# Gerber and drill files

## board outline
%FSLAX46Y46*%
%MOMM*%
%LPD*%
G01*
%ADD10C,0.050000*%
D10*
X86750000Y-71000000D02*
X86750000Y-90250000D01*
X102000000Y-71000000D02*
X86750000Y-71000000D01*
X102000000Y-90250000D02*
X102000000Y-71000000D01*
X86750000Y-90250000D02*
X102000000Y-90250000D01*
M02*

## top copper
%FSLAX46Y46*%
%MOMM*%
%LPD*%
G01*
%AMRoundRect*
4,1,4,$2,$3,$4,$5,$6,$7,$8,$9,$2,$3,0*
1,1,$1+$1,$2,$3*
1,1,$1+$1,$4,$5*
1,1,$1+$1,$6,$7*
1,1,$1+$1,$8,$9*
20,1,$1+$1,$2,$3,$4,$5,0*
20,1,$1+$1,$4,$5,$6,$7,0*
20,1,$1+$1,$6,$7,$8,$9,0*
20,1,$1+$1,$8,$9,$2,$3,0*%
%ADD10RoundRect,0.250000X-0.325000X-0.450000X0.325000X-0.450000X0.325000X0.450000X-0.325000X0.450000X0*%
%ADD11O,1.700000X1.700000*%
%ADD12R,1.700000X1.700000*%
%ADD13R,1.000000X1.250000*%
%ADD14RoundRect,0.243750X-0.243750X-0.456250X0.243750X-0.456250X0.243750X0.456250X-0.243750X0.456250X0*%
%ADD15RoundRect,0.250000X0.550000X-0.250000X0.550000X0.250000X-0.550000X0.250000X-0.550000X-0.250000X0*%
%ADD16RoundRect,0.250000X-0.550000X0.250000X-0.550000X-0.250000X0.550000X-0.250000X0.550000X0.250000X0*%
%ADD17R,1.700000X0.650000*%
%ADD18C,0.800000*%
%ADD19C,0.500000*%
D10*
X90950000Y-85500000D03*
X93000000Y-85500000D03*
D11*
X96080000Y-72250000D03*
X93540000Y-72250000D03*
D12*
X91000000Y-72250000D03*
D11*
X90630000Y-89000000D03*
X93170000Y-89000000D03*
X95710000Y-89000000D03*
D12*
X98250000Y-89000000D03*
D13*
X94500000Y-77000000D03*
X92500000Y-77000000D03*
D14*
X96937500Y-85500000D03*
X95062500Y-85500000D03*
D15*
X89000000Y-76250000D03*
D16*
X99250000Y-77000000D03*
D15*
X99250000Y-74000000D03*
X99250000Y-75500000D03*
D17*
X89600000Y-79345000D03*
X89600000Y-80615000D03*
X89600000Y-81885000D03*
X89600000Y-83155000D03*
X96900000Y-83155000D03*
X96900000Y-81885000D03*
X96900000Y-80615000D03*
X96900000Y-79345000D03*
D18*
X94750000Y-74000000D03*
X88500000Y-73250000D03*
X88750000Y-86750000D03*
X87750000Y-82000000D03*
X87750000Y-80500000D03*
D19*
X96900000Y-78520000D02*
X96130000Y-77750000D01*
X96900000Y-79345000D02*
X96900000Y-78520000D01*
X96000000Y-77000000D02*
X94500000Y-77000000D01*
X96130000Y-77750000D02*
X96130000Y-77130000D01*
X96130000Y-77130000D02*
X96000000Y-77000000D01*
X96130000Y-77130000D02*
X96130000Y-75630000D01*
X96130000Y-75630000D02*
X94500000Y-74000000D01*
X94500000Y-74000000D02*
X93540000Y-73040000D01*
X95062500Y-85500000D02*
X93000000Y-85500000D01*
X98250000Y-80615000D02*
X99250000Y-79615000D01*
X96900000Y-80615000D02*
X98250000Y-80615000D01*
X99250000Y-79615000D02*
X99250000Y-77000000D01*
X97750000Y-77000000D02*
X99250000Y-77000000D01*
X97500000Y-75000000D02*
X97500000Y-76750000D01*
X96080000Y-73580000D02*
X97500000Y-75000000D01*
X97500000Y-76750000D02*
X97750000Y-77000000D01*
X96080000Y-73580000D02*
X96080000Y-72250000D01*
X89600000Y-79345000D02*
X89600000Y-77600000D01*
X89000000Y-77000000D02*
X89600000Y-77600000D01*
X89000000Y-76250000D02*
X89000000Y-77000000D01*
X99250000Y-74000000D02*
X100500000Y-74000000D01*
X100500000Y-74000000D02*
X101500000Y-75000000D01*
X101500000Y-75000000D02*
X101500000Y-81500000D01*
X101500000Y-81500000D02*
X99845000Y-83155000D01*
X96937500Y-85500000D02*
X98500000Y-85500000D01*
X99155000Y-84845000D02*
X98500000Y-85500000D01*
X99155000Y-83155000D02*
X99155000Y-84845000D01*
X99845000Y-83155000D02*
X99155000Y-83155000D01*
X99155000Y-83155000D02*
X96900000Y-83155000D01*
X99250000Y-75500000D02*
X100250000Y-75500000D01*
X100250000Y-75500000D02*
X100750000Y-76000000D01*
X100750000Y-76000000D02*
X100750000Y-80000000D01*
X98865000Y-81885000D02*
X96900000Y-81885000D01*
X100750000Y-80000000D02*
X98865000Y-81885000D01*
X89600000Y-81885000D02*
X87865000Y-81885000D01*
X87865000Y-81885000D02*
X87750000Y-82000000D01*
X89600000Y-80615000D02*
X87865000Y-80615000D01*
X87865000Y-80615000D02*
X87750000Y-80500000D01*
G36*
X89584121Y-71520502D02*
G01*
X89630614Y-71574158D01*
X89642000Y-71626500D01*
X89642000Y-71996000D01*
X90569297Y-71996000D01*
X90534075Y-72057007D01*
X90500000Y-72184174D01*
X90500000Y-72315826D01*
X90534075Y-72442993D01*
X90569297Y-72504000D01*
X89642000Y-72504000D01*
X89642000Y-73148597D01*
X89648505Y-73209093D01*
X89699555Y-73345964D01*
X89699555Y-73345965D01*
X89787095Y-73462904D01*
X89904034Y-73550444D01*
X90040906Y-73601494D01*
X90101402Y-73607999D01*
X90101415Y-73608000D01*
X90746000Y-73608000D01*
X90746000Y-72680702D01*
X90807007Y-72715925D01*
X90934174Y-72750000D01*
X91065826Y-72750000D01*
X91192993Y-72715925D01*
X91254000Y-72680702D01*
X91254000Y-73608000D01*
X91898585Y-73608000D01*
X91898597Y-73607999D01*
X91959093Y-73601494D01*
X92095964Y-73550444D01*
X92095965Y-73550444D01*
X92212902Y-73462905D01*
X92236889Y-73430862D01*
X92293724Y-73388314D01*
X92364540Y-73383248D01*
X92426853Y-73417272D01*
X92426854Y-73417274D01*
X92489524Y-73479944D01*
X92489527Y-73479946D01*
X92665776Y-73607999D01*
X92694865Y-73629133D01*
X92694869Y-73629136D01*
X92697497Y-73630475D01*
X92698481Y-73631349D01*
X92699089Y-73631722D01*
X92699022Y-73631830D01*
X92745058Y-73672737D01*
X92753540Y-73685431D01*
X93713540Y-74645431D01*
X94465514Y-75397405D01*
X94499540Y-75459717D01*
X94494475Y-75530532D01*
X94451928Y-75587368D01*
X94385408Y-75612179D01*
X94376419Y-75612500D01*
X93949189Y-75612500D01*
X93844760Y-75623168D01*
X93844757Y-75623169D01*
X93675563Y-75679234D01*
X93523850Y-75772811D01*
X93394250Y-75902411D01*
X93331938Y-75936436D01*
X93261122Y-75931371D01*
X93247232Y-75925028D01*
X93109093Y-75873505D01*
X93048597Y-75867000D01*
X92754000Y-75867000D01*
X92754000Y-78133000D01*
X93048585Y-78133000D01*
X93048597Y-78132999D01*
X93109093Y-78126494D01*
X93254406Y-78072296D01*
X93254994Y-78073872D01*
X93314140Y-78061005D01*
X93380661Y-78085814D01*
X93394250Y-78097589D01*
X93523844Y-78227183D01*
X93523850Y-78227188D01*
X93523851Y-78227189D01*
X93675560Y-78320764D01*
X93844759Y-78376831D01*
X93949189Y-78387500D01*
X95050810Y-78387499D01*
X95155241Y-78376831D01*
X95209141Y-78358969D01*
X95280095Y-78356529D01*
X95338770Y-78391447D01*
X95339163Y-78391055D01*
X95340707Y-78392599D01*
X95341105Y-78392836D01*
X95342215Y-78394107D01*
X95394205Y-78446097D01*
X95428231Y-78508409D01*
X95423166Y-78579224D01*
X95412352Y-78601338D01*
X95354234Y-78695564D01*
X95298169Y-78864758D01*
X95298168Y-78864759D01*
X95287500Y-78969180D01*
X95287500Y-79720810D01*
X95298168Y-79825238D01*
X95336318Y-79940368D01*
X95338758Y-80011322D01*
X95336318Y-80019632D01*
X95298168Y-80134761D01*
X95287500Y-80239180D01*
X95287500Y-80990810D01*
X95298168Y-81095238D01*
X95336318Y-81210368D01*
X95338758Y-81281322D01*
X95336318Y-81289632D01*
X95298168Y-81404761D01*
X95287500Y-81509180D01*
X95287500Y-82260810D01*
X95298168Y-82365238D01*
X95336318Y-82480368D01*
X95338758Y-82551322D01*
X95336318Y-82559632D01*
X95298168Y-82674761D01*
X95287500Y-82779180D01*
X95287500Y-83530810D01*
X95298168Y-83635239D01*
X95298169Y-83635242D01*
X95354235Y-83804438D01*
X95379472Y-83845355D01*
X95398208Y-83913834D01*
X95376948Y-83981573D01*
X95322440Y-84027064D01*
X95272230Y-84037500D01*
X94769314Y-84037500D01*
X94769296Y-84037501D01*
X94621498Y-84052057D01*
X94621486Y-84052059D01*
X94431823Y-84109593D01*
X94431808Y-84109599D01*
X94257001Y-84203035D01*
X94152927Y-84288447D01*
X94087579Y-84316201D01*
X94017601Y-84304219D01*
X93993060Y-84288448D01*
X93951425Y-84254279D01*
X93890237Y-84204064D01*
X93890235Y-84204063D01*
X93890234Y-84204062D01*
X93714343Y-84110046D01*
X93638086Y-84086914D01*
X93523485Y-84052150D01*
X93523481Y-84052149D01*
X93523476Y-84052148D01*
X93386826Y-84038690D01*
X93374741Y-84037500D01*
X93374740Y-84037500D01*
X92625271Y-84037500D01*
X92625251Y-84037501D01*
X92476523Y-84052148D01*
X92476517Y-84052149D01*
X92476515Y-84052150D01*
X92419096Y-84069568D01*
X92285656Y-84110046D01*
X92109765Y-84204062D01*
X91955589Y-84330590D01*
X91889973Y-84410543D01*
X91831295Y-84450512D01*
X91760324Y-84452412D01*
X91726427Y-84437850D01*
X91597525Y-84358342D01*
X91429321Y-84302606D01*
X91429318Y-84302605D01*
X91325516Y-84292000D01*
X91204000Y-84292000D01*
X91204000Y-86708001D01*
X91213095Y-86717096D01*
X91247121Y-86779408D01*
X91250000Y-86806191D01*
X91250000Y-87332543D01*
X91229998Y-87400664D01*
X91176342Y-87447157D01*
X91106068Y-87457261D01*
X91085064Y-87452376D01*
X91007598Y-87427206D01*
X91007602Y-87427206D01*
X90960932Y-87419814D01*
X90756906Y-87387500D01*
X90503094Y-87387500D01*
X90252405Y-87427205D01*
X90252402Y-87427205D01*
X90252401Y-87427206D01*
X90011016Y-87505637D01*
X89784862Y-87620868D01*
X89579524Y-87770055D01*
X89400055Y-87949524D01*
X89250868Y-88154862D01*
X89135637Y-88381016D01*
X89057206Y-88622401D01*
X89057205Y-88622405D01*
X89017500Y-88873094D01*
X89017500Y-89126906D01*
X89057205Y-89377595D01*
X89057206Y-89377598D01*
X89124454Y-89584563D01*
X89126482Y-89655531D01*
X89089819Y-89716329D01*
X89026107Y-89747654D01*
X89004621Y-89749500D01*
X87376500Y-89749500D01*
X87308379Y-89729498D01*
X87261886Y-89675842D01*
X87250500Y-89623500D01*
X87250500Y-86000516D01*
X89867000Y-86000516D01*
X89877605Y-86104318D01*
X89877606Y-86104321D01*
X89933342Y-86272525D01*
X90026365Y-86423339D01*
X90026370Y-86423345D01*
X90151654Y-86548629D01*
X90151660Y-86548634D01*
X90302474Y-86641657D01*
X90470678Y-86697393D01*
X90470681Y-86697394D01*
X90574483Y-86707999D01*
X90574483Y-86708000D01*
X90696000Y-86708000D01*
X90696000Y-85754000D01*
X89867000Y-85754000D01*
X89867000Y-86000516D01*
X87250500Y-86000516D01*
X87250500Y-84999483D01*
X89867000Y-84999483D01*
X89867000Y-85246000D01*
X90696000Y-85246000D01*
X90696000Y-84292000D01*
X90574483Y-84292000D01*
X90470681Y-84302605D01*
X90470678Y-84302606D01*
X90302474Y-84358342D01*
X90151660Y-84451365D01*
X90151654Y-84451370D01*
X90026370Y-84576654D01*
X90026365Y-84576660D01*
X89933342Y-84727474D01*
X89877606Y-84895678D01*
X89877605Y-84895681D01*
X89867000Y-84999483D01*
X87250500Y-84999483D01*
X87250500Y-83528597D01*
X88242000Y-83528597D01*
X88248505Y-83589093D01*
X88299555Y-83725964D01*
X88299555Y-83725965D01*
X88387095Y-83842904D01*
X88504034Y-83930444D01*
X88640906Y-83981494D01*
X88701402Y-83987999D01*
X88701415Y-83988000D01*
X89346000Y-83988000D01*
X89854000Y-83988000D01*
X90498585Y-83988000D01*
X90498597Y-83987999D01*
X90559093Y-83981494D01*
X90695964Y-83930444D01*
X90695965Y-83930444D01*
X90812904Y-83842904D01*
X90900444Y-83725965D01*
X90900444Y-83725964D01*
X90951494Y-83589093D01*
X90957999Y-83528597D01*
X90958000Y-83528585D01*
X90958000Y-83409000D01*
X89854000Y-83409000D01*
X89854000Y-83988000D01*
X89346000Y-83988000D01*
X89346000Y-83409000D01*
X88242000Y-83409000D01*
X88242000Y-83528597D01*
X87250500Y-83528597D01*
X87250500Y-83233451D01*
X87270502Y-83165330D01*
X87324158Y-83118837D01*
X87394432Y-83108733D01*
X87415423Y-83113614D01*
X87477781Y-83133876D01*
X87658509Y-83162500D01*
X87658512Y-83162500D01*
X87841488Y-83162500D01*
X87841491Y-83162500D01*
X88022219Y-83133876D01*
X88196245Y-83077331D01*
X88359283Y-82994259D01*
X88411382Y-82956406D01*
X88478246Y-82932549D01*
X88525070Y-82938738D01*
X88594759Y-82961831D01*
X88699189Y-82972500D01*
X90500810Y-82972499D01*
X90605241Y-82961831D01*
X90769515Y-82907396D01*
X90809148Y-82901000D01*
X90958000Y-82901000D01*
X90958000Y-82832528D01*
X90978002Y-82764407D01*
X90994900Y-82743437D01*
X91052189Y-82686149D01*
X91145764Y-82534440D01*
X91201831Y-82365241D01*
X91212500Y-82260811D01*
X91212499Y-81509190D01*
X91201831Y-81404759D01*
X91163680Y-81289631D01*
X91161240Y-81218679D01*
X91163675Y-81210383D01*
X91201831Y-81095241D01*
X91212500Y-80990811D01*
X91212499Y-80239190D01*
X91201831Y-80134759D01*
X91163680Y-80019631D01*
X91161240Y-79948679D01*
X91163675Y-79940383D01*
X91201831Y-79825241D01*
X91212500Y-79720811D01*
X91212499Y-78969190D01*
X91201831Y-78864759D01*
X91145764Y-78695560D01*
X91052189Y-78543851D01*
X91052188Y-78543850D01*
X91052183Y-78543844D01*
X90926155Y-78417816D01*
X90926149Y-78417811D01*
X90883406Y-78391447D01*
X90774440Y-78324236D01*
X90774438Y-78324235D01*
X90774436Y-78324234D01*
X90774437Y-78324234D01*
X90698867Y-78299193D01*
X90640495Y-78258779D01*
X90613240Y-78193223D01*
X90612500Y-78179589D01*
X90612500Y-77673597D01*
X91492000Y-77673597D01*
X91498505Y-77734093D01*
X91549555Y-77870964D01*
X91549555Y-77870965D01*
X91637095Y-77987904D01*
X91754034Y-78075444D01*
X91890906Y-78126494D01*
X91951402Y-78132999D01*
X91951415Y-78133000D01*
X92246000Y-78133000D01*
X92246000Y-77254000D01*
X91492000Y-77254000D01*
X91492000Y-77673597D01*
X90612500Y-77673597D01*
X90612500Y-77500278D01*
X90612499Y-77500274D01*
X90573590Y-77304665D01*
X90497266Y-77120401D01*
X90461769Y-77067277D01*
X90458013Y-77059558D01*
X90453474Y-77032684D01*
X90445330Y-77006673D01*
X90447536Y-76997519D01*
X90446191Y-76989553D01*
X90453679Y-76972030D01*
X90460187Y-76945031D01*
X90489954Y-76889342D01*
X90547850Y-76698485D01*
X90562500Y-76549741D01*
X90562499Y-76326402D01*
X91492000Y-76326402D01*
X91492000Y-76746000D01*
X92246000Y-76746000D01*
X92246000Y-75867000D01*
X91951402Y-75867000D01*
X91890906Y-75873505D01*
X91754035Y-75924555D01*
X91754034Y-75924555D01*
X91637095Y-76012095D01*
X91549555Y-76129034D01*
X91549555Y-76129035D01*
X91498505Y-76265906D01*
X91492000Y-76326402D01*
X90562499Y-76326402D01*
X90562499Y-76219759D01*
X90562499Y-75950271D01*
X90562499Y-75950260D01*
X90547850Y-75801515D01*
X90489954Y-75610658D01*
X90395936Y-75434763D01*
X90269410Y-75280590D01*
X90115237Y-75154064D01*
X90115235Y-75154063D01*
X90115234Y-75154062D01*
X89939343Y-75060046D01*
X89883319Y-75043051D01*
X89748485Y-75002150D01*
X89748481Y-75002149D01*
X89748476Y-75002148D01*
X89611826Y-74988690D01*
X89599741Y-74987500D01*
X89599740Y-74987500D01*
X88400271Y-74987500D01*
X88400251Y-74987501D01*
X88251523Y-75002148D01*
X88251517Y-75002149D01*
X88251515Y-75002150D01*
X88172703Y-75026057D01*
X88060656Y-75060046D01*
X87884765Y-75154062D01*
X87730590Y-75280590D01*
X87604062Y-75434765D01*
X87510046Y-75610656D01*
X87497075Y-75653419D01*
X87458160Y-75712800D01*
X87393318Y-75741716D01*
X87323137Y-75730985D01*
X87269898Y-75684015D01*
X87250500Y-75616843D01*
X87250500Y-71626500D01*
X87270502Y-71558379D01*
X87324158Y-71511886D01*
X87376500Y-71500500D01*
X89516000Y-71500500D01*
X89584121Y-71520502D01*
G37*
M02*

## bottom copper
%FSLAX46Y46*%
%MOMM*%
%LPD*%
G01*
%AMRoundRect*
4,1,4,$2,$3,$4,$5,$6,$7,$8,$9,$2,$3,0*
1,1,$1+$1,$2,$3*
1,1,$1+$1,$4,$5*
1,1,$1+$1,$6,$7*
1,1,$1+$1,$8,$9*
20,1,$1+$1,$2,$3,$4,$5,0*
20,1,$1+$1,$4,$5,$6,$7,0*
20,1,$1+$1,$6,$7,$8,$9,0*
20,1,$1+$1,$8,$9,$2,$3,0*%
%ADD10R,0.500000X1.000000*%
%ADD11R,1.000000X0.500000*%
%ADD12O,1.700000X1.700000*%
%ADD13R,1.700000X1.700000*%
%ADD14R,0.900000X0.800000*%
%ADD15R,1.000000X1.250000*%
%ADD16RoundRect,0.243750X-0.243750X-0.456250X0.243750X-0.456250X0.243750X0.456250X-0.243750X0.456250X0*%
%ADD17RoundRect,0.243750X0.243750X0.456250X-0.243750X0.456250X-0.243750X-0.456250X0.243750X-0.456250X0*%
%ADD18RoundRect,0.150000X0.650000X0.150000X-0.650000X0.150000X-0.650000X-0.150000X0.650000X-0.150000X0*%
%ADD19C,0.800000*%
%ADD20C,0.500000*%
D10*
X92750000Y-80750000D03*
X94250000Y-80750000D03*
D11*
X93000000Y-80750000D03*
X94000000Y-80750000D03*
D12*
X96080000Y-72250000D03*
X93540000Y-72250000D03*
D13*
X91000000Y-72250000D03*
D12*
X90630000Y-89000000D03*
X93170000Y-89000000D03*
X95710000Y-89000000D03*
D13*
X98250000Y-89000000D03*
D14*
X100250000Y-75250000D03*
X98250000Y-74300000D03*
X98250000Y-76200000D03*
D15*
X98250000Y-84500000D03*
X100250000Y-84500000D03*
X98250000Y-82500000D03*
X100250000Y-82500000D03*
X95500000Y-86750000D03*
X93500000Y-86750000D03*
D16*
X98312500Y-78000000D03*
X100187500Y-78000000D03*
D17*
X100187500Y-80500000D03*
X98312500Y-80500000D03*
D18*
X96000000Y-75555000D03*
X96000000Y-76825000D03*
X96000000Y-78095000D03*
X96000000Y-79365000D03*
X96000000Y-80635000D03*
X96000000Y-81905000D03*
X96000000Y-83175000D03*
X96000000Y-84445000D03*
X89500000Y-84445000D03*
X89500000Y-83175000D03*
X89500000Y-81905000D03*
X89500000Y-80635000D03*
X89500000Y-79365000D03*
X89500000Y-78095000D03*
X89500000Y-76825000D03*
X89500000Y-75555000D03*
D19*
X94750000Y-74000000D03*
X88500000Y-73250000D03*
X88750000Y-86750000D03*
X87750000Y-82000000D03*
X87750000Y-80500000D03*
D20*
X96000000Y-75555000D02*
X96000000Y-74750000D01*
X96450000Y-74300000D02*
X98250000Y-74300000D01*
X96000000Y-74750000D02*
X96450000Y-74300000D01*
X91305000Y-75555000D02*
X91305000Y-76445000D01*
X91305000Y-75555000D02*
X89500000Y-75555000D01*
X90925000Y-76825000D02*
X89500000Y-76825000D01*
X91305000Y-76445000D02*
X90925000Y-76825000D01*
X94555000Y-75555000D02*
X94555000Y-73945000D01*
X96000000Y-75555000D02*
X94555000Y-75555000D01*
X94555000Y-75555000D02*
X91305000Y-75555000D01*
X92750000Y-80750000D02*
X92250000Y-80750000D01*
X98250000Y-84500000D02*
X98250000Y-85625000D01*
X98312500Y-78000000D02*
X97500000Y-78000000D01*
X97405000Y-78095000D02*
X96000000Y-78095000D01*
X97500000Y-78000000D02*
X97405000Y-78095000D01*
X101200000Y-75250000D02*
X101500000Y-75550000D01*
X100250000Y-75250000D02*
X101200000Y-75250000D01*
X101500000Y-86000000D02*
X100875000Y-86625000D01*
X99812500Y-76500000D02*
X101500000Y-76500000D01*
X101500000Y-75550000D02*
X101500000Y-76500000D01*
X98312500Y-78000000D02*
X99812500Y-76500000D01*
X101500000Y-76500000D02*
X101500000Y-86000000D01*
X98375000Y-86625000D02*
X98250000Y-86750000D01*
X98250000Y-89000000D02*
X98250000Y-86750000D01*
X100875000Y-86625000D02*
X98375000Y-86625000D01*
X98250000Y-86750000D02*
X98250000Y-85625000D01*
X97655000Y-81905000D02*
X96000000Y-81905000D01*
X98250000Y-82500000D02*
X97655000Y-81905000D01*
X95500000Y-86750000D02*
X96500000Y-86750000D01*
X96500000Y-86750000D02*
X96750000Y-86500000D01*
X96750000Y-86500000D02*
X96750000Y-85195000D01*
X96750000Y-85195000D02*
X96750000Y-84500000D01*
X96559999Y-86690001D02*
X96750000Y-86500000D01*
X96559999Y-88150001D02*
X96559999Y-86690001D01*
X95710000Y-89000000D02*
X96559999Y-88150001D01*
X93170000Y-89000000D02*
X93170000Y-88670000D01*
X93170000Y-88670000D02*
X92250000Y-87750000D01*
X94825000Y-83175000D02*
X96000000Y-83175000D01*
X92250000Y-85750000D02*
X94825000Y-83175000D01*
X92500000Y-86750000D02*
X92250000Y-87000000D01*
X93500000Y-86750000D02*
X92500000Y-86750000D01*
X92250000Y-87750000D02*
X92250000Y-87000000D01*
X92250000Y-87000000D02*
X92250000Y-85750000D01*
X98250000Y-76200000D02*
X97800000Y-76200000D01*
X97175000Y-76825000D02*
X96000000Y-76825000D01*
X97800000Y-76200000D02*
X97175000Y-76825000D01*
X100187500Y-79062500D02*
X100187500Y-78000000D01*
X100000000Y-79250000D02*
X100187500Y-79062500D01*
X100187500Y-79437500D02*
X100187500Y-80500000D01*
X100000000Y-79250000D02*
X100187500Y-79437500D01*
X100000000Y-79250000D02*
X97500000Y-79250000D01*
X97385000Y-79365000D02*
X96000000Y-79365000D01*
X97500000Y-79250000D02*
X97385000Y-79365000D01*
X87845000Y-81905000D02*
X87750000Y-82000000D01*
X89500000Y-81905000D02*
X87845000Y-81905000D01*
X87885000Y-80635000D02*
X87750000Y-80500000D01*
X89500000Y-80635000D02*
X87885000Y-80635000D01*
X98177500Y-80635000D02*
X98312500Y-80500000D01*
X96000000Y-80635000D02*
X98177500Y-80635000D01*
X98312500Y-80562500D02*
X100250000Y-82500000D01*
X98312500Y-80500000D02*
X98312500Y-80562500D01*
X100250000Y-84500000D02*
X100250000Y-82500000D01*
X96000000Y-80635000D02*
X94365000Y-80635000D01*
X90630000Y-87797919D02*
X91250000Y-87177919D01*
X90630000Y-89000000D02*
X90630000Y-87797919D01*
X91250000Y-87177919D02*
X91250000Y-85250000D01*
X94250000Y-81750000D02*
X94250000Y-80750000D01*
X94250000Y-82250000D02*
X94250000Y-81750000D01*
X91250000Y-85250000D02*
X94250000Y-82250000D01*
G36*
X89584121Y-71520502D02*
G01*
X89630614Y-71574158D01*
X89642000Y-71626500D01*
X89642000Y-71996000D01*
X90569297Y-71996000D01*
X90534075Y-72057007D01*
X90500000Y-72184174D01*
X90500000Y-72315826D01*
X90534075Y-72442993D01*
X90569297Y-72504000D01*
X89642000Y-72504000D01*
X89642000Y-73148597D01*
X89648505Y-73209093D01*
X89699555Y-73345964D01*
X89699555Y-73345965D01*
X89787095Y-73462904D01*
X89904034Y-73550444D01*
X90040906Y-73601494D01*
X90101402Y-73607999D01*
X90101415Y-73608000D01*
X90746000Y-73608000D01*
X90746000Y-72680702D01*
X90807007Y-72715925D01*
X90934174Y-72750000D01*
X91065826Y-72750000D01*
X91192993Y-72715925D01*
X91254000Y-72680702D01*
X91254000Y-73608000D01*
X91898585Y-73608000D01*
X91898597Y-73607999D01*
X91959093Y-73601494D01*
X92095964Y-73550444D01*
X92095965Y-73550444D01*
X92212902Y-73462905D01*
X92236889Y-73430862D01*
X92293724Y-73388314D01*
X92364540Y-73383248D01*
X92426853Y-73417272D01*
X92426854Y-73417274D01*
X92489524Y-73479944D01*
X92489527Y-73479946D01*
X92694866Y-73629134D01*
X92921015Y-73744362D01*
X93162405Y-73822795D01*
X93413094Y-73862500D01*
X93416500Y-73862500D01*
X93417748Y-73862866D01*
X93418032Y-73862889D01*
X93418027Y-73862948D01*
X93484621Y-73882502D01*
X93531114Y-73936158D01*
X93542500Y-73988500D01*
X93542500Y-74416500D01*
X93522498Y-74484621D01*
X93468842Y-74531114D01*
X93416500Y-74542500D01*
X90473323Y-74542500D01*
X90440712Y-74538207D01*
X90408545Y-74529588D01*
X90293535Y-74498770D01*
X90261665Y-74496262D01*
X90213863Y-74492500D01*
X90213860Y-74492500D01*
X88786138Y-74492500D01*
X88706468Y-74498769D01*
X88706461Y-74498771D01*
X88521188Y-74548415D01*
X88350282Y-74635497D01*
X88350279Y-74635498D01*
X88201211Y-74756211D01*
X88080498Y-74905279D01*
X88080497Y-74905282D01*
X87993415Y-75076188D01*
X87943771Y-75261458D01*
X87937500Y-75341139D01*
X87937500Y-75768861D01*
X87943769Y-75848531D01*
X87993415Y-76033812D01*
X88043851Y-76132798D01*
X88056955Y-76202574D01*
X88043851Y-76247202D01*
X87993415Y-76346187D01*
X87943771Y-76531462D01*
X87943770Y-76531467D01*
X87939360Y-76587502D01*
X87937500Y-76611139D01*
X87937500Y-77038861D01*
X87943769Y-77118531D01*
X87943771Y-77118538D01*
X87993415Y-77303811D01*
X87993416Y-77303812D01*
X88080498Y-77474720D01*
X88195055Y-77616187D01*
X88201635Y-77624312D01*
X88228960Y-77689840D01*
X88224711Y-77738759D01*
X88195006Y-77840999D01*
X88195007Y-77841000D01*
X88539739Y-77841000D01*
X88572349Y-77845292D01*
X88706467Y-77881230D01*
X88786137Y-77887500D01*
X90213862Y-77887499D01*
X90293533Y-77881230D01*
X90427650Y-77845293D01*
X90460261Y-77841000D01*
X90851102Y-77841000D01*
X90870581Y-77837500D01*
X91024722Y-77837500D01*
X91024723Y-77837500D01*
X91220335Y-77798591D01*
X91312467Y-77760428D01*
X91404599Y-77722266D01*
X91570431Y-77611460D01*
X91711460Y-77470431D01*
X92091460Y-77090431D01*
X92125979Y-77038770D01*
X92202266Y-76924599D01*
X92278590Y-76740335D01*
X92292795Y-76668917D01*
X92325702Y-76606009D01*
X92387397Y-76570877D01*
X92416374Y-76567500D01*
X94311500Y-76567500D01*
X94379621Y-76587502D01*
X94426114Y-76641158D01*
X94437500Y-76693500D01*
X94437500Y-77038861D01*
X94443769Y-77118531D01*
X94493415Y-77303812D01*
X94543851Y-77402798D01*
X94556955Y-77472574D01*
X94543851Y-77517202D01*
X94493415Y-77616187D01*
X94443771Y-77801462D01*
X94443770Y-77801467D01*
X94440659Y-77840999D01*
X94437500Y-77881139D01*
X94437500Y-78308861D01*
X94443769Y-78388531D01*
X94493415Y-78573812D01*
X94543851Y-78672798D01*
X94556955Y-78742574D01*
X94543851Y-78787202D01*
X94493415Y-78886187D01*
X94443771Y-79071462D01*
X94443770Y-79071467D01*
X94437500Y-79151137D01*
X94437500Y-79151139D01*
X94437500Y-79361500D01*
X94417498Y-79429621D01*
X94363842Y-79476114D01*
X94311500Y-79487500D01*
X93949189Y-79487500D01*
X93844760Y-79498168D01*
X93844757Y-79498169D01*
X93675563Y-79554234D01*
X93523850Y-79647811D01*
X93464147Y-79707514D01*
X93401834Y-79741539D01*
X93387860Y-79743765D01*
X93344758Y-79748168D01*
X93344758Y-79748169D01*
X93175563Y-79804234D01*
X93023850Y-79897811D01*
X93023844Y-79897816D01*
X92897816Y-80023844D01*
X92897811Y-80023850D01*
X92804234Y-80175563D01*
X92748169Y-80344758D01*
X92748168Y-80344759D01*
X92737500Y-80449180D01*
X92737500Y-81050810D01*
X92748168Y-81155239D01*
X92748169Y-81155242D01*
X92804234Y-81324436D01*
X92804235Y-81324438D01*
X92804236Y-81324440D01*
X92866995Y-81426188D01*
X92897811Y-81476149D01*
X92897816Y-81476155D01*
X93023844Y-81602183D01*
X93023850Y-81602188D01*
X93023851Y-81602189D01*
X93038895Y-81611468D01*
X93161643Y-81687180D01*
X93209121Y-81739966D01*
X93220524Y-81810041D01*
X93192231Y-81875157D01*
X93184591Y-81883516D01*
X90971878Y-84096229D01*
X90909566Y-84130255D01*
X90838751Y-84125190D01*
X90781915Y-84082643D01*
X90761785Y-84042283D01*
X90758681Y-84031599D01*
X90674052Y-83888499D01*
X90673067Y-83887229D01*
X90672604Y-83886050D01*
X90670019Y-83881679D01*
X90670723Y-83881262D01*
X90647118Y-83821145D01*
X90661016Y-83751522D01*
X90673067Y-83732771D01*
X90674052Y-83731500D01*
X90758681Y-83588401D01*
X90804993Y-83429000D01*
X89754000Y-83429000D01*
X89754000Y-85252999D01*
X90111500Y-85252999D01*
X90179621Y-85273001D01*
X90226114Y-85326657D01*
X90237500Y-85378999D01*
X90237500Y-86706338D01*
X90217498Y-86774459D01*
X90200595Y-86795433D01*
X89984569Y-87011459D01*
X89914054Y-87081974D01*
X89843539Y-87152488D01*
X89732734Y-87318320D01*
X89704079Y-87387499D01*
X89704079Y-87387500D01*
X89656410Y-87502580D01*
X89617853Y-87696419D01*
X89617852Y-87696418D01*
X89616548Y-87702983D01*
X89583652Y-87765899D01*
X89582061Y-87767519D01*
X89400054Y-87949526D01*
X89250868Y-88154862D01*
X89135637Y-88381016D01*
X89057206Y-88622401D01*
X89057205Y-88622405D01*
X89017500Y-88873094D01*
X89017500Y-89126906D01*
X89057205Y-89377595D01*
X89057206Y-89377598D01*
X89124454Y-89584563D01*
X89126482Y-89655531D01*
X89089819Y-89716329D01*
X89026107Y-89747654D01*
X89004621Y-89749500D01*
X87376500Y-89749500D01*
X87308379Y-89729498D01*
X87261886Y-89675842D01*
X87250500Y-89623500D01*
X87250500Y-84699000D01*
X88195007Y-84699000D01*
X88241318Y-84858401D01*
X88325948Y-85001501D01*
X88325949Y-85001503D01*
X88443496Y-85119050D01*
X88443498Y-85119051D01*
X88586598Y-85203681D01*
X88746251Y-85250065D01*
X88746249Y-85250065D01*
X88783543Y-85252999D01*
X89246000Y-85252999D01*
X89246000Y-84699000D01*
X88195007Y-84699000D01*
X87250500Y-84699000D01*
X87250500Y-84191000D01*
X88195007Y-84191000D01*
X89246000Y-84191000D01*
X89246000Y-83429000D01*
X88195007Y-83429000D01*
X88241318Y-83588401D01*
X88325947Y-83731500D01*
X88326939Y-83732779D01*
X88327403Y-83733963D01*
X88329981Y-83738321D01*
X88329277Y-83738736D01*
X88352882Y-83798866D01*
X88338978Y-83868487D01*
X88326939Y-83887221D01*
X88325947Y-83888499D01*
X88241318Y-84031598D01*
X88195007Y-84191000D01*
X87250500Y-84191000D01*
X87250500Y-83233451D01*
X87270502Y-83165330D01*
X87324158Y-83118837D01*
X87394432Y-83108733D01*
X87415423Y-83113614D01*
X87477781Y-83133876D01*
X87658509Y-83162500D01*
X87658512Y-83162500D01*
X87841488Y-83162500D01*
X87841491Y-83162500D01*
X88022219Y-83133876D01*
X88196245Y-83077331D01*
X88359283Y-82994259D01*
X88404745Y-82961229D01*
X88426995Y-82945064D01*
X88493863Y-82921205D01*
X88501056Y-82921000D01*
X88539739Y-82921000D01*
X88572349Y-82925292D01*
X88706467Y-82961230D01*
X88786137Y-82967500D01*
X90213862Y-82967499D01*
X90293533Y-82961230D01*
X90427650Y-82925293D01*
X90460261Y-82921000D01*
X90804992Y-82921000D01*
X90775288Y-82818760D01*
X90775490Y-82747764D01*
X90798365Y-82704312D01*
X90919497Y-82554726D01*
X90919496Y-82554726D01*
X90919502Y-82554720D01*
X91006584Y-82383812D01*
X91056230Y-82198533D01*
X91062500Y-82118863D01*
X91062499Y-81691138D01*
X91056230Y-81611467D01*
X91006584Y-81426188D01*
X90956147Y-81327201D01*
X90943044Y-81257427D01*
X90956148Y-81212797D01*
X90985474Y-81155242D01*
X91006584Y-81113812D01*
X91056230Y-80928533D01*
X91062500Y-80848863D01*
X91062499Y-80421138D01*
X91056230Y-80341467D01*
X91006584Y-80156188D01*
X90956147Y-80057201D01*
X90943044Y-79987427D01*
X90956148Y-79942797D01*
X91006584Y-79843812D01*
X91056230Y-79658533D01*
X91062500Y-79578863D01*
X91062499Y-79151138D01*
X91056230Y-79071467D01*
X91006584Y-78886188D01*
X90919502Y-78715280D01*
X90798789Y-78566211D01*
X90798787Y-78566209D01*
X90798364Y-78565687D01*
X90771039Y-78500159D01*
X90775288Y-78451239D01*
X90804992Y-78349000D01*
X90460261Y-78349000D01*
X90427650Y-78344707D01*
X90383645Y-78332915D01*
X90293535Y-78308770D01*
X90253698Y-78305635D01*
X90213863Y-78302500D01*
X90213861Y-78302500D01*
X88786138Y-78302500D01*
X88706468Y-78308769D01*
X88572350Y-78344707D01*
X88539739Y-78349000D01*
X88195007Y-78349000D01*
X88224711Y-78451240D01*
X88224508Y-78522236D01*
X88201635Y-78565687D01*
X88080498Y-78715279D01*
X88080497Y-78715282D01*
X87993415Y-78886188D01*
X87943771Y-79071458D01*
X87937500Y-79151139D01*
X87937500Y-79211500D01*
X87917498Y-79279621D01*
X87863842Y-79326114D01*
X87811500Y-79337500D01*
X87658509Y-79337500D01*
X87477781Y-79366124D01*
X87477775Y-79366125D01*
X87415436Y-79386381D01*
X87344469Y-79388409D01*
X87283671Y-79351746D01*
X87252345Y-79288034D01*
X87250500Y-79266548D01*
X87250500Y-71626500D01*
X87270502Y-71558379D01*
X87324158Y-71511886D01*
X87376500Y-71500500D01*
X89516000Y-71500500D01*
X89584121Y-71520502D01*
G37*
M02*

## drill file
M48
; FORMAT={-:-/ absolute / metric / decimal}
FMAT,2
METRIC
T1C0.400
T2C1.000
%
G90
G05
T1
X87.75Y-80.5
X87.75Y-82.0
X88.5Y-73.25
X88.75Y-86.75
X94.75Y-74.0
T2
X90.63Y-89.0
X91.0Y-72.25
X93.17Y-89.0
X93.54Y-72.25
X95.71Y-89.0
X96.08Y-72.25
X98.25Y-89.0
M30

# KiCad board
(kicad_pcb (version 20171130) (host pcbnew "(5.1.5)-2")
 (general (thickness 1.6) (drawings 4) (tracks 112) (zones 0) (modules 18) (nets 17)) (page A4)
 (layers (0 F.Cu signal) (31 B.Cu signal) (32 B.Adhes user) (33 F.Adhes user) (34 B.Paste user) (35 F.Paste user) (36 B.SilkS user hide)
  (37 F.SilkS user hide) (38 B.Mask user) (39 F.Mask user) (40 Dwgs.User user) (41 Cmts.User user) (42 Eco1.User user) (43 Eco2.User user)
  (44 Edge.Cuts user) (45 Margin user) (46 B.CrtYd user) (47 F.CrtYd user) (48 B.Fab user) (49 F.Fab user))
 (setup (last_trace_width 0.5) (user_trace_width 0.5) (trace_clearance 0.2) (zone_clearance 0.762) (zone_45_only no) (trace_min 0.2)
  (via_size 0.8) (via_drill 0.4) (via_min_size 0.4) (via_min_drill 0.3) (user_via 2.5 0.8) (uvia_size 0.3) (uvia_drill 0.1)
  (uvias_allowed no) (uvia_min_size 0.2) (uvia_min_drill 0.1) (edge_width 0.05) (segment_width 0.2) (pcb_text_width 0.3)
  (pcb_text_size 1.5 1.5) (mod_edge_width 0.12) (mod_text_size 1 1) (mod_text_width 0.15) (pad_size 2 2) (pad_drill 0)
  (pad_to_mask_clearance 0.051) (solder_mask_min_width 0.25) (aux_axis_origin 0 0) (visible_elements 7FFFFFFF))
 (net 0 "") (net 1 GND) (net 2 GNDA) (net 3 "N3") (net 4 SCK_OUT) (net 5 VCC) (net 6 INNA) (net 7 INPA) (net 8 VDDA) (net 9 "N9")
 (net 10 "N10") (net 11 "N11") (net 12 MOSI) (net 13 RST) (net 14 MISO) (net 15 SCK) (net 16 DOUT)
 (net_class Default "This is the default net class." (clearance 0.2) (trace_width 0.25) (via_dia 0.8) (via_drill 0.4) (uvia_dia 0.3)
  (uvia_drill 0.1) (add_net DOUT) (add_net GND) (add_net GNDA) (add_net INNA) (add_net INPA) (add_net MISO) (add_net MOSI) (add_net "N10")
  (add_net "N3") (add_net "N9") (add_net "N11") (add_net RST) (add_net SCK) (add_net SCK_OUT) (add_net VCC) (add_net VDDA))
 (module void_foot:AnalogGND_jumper (layer B.Cu) (at 93.5 80.75 180) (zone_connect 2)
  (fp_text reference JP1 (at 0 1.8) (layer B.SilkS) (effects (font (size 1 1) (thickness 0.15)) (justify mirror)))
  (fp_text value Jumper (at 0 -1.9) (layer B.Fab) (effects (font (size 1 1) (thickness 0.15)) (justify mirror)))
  (pad 2 smd rect (at 0.75 0 180) (size 0.5 1) (layers B.Cu B.Mask) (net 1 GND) (zone_connect 2))
  (pad 1 smd rect (at -0.75 0 180) (size 0.5 1) (layers B.Cu B.Mask) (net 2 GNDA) (zone_connect 2))
  (pad 2 smd rect (at 0.5 0 180) (size 1 0.5) (layers B.Cu B.Mask) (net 1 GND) (zone_connect 2))
  (pad 1 smd rect (at -0.5 0 180) (size 1 0.5) (layers B.Cu B.Mask) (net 2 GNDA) (zone_connect 2)))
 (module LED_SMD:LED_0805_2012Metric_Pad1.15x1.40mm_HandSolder (layer F.Cu) (at 91.975 85.5)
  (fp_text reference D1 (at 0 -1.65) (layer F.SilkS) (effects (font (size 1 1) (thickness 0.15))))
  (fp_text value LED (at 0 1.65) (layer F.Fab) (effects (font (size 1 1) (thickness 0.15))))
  (pad 1 smd roundrect (at -1.025 0) (size 1.15 1.4) (layers F.Cu F.Paste F.Mask) (roundrect_rratio 0.217391) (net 1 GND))
  (pad 2 smd roundrect (at 1.025 0) (size 1.15 1.4) (layers F.Cu F.Paste F.Mask) (roundrect_rratio 0.217391) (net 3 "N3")))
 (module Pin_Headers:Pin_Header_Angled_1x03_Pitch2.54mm (layer F.Cu) (at 91 72.25 90)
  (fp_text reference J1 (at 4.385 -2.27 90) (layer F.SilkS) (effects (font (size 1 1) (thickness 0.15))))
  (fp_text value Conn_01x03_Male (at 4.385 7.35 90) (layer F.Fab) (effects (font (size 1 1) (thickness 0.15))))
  (pad 3 thru_hole oval (at 0 5.08 90) (size 1.7 1.7) (drill 1) (layers *.Cu *.Mask) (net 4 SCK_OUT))
  (pad 2 thru_hole oval (at 0 2.54 90) (size 1.7 1.7) (drill 1) (layers *.Cu *.Mask) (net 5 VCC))
  (pad 1 thru_hole rect (at 0 0 90) (size 1.7 1.7) (drill 1) (layers *.Cu *.Mask) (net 1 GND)))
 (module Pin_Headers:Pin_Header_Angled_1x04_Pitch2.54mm (layer F.Cu) (at 98.25 89 270)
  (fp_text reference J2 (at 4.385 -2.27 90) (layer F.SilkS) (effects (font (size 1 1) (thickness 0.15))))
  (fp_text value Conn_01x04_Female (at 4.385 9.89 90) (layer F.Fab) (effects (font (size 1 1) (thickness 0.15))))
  (pad 4 thru_hole oval (at 0 7.62 270) (size 1.7 1.7) (drill 1) (layers *.Cu *.Mask) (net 2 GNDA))
  (pad 3 thru_hole oval (at 0 5.08 270) (size 1.7 1.7) (drill 1) (layers *.Cu *.Mask) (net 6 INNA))
  (pad 2 thru_hole oval (at 0 2.54 270) (size 1.7 1.7) (drill 1) (layers *.Cu *.Mask) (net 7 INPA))
  (pad 1 thru_hole rect (at 0 0 270) (size 1.7 1.7) (drill 1) (layers *.Cu *.Mask) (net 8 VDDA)))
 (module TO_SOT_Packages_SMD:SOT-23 (layer B.Cu) (at 99.25 75.25)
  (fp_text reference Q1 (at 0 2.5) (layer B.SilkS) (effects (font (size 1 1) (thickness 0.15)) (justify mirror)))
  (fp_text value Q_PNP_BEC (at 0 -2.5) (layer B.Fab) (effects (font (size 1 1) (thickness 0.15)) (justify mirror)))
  (pad 3 smd rect (at 1 0) (size 0.9 0.8) (layers B.Cu B.Paste B.Mask) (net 8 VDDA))
  (pad 2 smd rect (at -1 -0.95) (size 0.9 0.8) (layers B.Cu B.Paste B.Mask) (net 5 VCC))
  (pad 1 smd rect (at -1 0.95) (size 0.9 0.8) (layers B.Cu B.Paste B.Mask) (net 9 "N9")))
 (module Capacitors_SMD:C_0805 (layer F.Cu) (at 93.5 77 180)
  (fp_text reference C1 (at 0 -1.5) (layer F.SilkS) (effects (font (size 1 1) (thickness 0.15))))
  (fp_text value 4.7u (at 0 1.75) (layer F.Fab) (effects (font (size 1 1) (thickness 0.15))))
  (pad 1 smd rect (at -1 0 180) (size 1 1.25) (layers F.Cu F.Paste F.Mask) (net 5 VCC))
  (pad 2 smd rect (at 1 0 180) (size 1 1.25) (layers F.Cu F.Paste F.Mask) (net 1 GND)))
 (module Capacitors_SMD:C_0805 (layer B.Cu) (at 99.25 84.5)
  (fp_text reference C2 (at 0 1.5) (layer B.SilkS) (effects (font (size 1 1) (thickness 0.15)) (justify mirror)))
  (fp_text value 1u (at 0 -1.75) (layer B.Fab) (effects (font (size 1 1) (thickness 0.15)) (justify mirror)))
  (pad 1 smd rect (at -1 0) (size 1 1.25) (layers B.Cu B.Paste B.Mask) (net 8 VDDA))
  (pad 2 smd rect (at 1 0) (size 1 1.25) (layers B.Cu B.Paste B.Mask) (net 2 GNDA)))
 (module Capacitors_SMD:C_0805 (layer B.Cu) (at 99.25 82.5 180)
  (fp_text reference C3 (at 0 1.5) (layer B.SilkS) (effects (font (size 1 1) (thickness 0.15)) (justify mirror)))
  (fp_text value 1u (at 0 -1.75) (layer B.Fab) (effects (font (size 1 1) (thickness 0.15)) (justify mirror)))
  (pad 2 smd rect (at 1 0 180) (size 1 1.25) (layers B.Cu B.Paste B.Mask) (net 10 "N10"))
  (pad 1 smd rect (at -1 0 180) (size 1 1.25) (layers B.Cu B.Paste B.Mask) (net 2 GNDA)))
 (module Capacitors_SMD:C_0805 (layer B.Cu) (at 94.5 86.75)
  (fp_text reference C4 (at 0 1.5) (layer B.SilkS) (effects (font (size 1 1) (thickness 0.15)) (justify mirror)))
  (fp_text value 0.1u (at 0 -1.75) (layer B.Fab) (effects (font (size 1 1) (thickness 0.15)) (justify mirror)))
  (pad 2 smd rect (at 1 0) (size 1 1.25) (layers B.Cu B.Paste B.Mask) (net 7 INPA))
  (pad 1 smd rect (at -1 0) (size 1 1.25) (layers B.Cu B.Paste B.Mask) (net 6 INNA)))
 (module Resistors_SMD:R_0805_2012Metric (layer B.Cu) (at 99.25 78)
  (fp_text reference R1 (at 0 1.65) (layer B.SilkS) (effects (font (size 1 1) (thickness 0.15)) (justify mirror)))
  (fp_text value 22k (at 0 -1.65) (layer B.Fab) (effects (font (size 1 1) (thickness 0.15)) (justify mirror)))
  (pad 1 smd roundrect (at -0.9375 0) (size 0.975 1.4) (layers B.Cu B.Paste B.Mask) (roundrect_rratio 0.25) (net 8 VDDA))
  (pad 2 smd roundrect (at 0.9375 0) (size 0.975 1.4) (layers B.Cu B.Paste B.Mask) (roundrect_rratio 0.25) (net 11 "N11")))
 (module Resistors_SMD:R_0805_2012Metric (layer B.Cu) (at 99.25 80.5 180)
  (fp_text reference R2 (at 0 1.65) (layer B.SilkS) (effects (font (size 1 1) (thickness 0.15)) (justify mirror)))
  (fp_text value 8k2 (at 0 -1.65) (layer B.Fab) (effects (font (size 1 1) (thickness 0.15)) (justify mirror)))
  (pad 1 smd roundrect (at -0.9375 0 180) (size 0.975 1.4) (layers B.Cu B.Paste B.Mask) (roundrect_rratio 0.25) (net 11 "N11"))
  (pad 2 smd roundrect (at 0.9375 0 180) (size 0.975 1.4) (layers B.Cu B.Paste B.Mask) (roundrect_rratio 0.25) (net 2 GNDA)))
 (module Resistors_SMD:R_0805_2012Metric (layer F.Cu) (at 96 85.5)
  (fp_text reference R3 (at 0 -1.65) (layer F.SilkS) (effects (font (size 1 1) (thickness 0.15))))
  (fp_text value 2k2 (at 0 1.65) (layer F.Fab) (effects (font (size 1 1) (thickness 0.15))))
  (pad 2 smd roundrect (at 0.9375 0) (size 0.975 1.4) (layers F.Cu F.Paste F.Mask) (roundrect_rratio 0.25) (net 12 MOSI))
  (pad 1 smd roundrect (at -0.9375 0) (size 0.975 1.4) (layers F.Cu F.Paste F.Mask) (roundrect_rratio 0.25) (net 3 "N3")))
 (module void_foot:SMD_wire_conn (layer F.Cu) (at 89 76.25 90)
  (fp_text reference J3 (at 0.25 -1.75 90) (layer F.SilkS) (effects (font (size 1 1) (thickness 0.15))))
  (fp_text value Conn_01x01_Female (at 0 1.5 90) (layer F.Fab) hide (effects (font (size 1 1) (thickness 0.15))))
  (pad 1 smd roundrect (at 0 0 90) (size 1 1.6) (layers F.Cu F.Paste F.Mask) (roundrect_rratio 0.25) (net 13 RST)))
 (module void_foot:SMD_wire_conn (layer F.Cu) (at 99.25 77 270)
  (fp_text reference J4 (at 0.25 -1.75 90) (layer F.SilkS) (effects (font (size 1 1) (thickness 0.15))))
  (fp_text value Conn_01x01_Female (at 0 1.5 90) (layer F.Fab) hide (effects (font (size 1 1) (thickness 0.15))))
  (pad 1 smd roundrect (at 0 0 270) (size 1 1.6) (layers F.Cu F.Paste F.Mask) (roundrect_rratio 0.25) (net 4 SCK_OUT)))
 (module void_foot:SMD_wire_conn (layer F.Cu) (at 99.25 74 90)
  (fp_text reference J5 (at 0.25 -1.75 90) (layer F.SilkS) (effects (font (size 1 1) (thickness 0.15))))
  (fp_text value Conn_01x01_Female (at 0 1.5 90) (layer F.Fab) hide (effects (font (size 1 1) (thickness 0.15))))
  (pad 1 smd roundrect (at 0 0 90) (size 1 1.6) (layers F.Cu F.Paste F.Mask) (roundrect_rratio 0.25) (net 12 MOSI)))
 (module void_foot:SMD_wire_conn (layer F.Cu) (at 99.25 75.5 90)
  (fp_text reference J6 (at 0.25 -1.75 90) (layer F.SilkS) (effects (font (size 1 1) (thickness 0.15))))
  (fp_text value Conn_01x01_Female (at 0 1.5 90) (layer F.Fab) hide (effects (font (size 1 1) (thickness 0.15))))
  (pad 1 smd roundrect (at 0 0 90) (size 1 1.6) (layers F.Cu F.Paste F.Mask) (roundrect_rratio 0.25) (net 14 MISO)))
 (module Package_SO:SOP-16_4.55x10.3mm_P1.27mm (layer B.Cu) (at 92.75 80 180)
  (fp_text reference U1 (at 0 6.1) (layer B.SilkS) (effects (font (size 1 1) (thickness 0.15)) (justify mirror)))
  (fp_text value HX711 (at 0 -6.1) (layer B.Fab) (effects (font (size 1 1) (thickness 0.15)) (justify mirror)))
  (pad 1 smd roundrect (at -3.25 4.445 180) (size 1.6 0.6) (layers B.Cu B.Paste B.Mask) (roundrect_rratio 0.25) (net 5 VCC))
  (pad 2 smd roundrect (at -3.25 3.175 180) (size 1.6 0.6) (layers B.Cu B.Paste B.Mask) (roundrect_rratio 0.25) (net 9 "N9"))
  (pad 3 smd roundrect (at -3.25 1.905 180) (size 1.6 0.6) (layers B.Cu B.Paste B.Mask) (roundrect_rratio 0.25) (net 8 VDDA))
  (pad 4 smd roundrect (at -3.25 0.635 180) (size 1.6 0.6) (layers B.Cu B.Paste B.Mask) (roundrect_rratio 0.25) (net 11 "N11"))
  (pad 5 smd roundrect (at -3.25 -0.635 180) (size 1.6 0.6) (layers B.Cu B.Paste B.Mask) (roundrect_rratio 0.25) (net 2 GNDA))
  (pad 6 smd roundrect (at -3.25 -1.905 180) (size 1.6 0.6) (layers B.Cu B.Paste B.Mask) (roundrect_rratio 0.25) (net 10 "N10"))
  (pad 7 smd roundrect (at -3.25 -3.175 180) (size 1.6 0.6) (layers B.Cu B.Paste B.Mask) (roundrect_rratio 0.25) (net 6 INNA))
  (pad 8 smd roundrect (at -3.25 -4.445 180) (size 1.6 0.6) (layers B.Cu B.Paste B.Mask) (roundrect_rratio 0.25) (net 7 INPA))
  (pad 9 smd roundrect (at 3.25 -4.445 180) (size 1.6 0.6) (layers B.Cu B.Paste B.Mask) (roundrect_rratio 0.25) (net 1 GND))
  (pad 10 smd roundrect (at 3.25 -3.175 180) (size 1.6 0.6) (layers B.Cu B.Paste B.Mask) (roundrect_rratio 0.25) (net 1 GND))
  (pad 11 smd roundrect (at 3.25 -1.905 180) (size 1.6 0.6) (layers B.Cu B.Paste B.Mask) (roundrect_rratio 0.25) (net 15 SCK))
  (pad 12 smd roundrect (at 3.25 -0.635 180) (size 1.6 0.6) (layers B.Cu B.Paste B.Mask) (roundrect_rratio 0.25) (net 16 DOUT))
  (pad 13 smd roundrect (at 3.25 0.635 180) (size 1.6 0.6) (layers B.Cu B.Paste B.Mask) (roundrect_rratio 0.25))
  (pad 14 smd roundrect (at 3.25 1.905 180) (size 1.6 0.6) (layers B.Cu B.Paste B.Mask) (roundrect_rratio 0.25) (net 1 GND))
  (pad 15 smd roundrect (at 3.25 3.175 180) (size 1.6 0.6) (layers B.Cu B.Paste B.Mask) (roundrect_rratio 0.25) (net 5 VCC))
  (pad 16 smd roundrect (at 3.25 4.445 180) (size 1.6 0.6) (layers B.Cu B.Paste B.Mask) (roundrect_rratio 0.25) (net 5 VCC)))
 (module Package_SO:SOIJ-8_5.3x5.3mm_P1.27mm (layer F.Cu) (at 93.25 81.25)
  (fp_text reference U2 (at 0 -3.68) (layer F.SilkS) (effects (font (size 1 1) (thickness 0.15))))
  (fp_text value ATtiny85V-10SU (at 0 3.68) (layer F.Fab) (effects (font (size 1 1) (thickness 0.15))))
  (pad 1 smd rect (at -3.65 -1.905) (size 1.7 0.65) (layers F.Cu F.Paste F.Mask) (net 13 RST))
  (pad 2 smd rect (at -3.65 -0.635) (size 1.7 0.65) (layers F.Cu F.Paste F.Mask) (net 16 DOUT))
  (pad 3 smd rect (at -3.65 0.635) (size 1.7 0.65) (layers F.Cu F.Paste F.Mask) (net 15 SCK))
  (pad 4 smd rect (at -3.65 1.905) (size 1.7 0.65) (layers F.Cu F.Paste F.Mask) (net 1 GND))
  (pad 5 smd rect (at 3.65 1.905) (size 1.7 0.65) (layers F.Cu F.Paste F.Mask) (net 12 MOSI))
  (pad 6 smd rect (at 3.65 0.635) (size 1.7 0.65) (layers F.Cu F.Paste F.Mask) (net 14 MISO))
  (pad 7 smd rect (at 3.65 -0.635) (size 1.7 0.65) (layers F.Cu F.Paste F.Mask) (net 4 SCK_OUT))
  (pad 8 smd rect (at 3.65 -1.905) (size 1.7 0.65) (layers F.Cu F.Paste F.Mask) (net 5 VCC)))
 (gr_line (start 86.75 71) (end 86.75 90.25) (layer Edge.Cuts) (width 0.05))
 (gr_line (start 102 71) (end 86.75 71) (layer Edge.Cuts) (width 0.05))
 (gr_line (start 102 90.25) (end 102 71) (layer Edge.Cuts) (width 0.05))
 (gr_line (start 86.75 90.25) (end 102 90.25) (layer Edge.Cuts) (width 0.05))
 (segment (start 96.9 78.52) (end 96.13 77.75) (width 0.5) (layer F.Cu) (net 5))
 (segment (start 96.9 79.345) (end 96.9 78.52) (width 0.5) (layer F.Cu) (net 5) (status 10))
 (segment (start 96 77) (end 94.5 77) (width 0.5) (layer F.Cu) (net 5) (status 20))
 (segment (start 96.13 77.75) (end 96.13 77.13) (width 0.5) (layer F.Cu) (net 5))
 (segment (start 96.13 77.13) (end 96 77) (width 0.5) (layer F.Cu) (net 5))
 (segment (start 96.13 77.13) (end 96.13 75.63) (width 0.5) (layer F.Cu) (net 5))
 (segment (start 96 75.555) (end 96 74.75) (width 0.5) (layer B.Cu) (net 5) (status 10))
 (segment (start 96.45 74.3) (end 98.25 74.3) (width 0.5) (layer B.Cu) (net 5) (status 20))
 (segment (start 96 74.75) (end 96.45 74.3) (width 0.5) (layer B.Cu) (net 5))
 (segment (start 91.305 75.555) (end 91.305 76.445) (width 0.5) (layer B.Cu) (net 5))
 (segment (start 91.305 75.555) (end 89.5 75.555) (width 0.5) (layer B.Cu) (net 5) (status 20))
 (segment (start 90.925 76.825) (end 89.5 76.825) (width 0.5) (layer B.Cu) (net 5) (status 20))
 (segment (start 91.305 76.445) (end 90.925 76.825) (width 0.5) (layer B.Cu) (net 5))
 (via (at 94.75 74) (size 0.8) (drill 0.4) (layers F.Cu B.Cu) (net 5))
 (segment (start 94.555 75.555) (end 94.555 73.945) (width 0.5) (layer B.Cu) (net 5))
 (segment (start 96 75.555) (end 94.555 75.555) (width 0.5) (layer B.Cu) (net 5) (status 10))
 (segment (start 94.555 75.555) (end 91.305 75.555) (width 0.5) (layer B.Cu) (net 5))
 (segment (start 96.13 75.63) (end 94.5 74) (width 0.5) (layer F.Cu) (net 5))
 (segment (start 94.5 74) (end 93.54 73.04) (width 0.5) (layer F.Cu) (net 5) (status 20))
 (via (at 88.5 73.25) (size 0.8) (drill 0.4) (layers F.Cu B.Cu) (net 1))
 (segment (start 92.75 80.75) (end 92.25 80.75) (width 0.5) (layer B.Cu) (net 1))
 (via (at 88.75 86.75) (size 0.8) (drill 0.4) (layers F.Cu B.Cu) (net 1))
 (segment (start 98.25 84.5) (end 98.25 85.625) (width 0.5) (layer B.Cu) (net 8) (status 10))
 (segment (start 98.3125 78) (end 97.5 78) (width 0.5) (layer B.Cu) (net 8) (status 10))
 (segment (start 97.405 78.095) (end 96 78.095) (width 0.5) (layer B.Cu) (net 8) (status 20))
 (segment (start 97.5 78) (end 97.405 78.095) (width 0.5) (layer B.Cu) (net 8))
 (segment (start 101.2 75.25) (end 101.5 75.55) (width 0.5) (layer B.Cu) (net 8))
 (segment (start 100.25 75.25) (end 101.2 75.25) (width 0.5) (layer B.Cu) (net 8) (status 10))
 (segment (start 101.5 86) (end 100.875 86.625) (width 0.5) (layer B.Cu) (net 8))
 (segment (start 99.8125 76.5) (end 101.5 76.5) (width 0.5) (layer B.Cu) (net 8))
 (segment (start 101.5 75.55) (end 101.5 76.5) (width 0.5) (layer B.Cu) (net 8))
 (segment (start 98.3125 78) (end 99.8125 76.5) (width 0.5) (layer B.Cu) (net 8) (status 10))
 (segment (start 101.5 76.5) (end 101.5 86) (width 0.5) (layer B.Cu) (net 8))
 (segment (start 98.375 86.625) (end 98.25 86.75) (width 0.5) (layer B.Cu) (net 8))
 (segment (start 98.25 89) (end 98.25 86.75) (width 0.5) (layer B.Cu) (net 8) (status 10))
 (segment (start 100.875 86.625) (end 98.375 86.625) (width 0.5) (layer B.Cu) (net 8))
 (segment (start 98.25 86.75) (end 98.25 85.625) (width 0.5) (layer B.Cu) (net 8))
 (segment (start 97.655 81.905) (end 96 81.905) (width 0.5) (layer B.Cu) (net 10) (status 20))
 (segment (start 98.25 82.5) (end 97.655 81.905) (width 0.5) (layer B.Cu) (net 10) (status 10))
 (segment (start 95.5 86.75) (end 96.5 86.75) (width 0.5) (layer B.Cu) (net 7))
 (segment (start 96.5 86.75) (end 96.75 86.5) (width 0.5) (layer B.Cu) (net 7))
 (segment (start 96.75 86.5) (end 96.75 85.195) (width 0.5) (layer B.Cu) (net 7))
 (segment (start 96.75 85.195) (end 96.75 84.5) (width 0.5) (layer B.Cu) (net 7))
 (segment (start 96.559999 86.690001) (end 96.75 86.5) (width 0.5) (layer B.Cu) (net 7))
 (segment (start 96.559999 88.150001) (end 96.559999 86.690001) (width 0.5) (layer B.Cu) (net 7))
 (segment (start 95.71 89) (end 96.559999 88.150001) (width 0.5) (layer B.Cu) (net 7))
 (segment (start 93.17 89) (end 93.17 88.67) (width 0.5) (layer B.Cu) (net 6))
 (segment (start 93.17 88.67) (end 92.25 87.75) (width 0.5) (layer B.Cu) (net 6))
 (segment (start 94.825 83.175) (end 96 83.175) (width 0.5) (layer B.Cu) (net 6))
 (segment (start 92.25 85.75) (end 94.825 83.175) (width 0.5) (layer B.Cu) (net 6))
 (segment (start 92.5 86.75) (end 92.25 87) (width 0.5) (layer B.Cu) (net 6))
 (segment (start 93.5 86.75) (end 92.5 86.75) (width 0.5) (layer B.Cu) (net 6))
 (segment (start 92.25 87.75) (end 92.25 87) (width 0.5) (layer B.Cu) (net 6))
 (segment (start 92.25 87) (end 92.25 85.75) (width 0.5) (layer B.Cu) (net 6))
 (segment (start 95.0625 85.5) (end 93 85.5) (width 0.5) (layer F.Cu) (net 3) (status 30))
 (segment (start 98.25 80.615) (end 99.25 79.615) (width 0.5) (layer F.Cu) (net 4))
 (segment (start 96.9 80.615) (end 98.25 80.615) (width 0.5) (layer F.Cu) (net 4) (status 10))
 (segment (start 99.25 79.615) (end 99.25 77) (width 0.5) (layer F.Cu) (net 4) (status 20))
 (segment (start 97.75 77) (end 99.25 77) (width 0.5) (layer F.Cu) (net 4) (status 20))
 (segment (start 97.5 75) (end 97.5 76.75) (width 0.5) (layer F.Cu) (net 4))
 (segment (start 96.08 73.58) (end 97.5 75) (width 0.5) (layer F.Cu) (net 4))
 (segment (start 97.5 76.75) (end 97.75 77) (width 0.5) (layer F.Cu) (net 4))
 (segment (start 96.08 73.58) (end 96.08 72.25) (width 0.5) (layer F.Cu) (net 4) (status 20))
 (segment (start 89.6 79.345) (end 89.6 77.6) (width 0.5) (layer F.Cu) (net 13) (status 30))
 (segment (start 89 77) (end 89.6 77.6) (width 0.5) (layer F.Cu) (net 13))
 (segment (start 89 76.25) (end 89 77) (width 0.5) (layer F.Cu) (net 13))
 (segment (start 99.25 74) (end 100.5 74) (width 0.5) (layer F.Cu) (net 12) (status 10))
 (segment (start 100.5 74) (end 101.5 75) (width 0.5) (layer F.Cu) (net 12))
 (segment (start 101.5 75) (end 101.5 81.5) (width 0.5) (layer F.Cu) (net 12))
 (segment (start 101.5 81.5) (end 99.845 83.155) (width 0.5) (layer F.Cu) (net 12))
 (segment (start 96.9375 85.5) (end 98.5 85.5) (width 0.5) (layer F.Cu) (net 12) (status 10))
 (segment (start 99.155 84.845) (end 98.5 85.5) (width 0.5) (layer F.Cu) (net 12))
 (segment (start 99.155 83.155) (end 99.155 84.845) (width 0.5) (layer F.Cu) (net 12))
 (segment (start 99.845 83.155) (end 99.155 83.155) (width 0.5) (layer F.Cu) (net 12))
 (segment (start 99.155 83.155) (end 96.9 83.155) (width 0.5) (layer F.Cu) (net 12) (status 20))
 (segment (start 99.25 75.5) (end 100.25 75.5) (width 0.5) (layer F.Cu) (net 14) (status 10))
 (segment (start 100.25 75.5) (end 100.75 76) (width 0.5) (layer F.Cu) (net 14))
 (segment (start 100.75 76) (end 100.75 80) (width 0.5) (layer F.Cu) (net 14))
 (segment (start 98.865 81.885) (end 96.9 81.885) (width 0.5) (layer F.Cu) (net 14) (status 20))
 (segment (start 100.75 80) (end 98.865 81.885) (width 0.5) (layer F.Cu) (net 14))
 (segment (start 98.25 76.2) (end 97.8 76.2) (width 0.5) (layer B.Cu) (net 9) (status 30))
 (segment (start 97.175 76.825) (end 96 76.825) (width 0.5) (layer B.Cu) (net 9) (status 20))
 (segment (start 97.8 76.2) (end 97.175 76.825) (width 0.5) (layer B.Cu) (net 9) (status 10))
 (segment (start 100.1875 79.0625) (end 100.1875 78) (width 0.5) (layer B.Cu) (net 11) (status 20))
 (segment (start 100 79.25) (end 100.1875 79.0625) (width 0.5) (layer B.Cu) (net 11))
 (segment (start 100.1875 79.4375) (end 100.1875 80.5) (width 0.5) (layer B.Cu) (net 11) (status 20))
 (segment (start 100 79.25) (end 100.1875 79.4375) (width 0.5) (layer B.Cu) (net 11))
 (segment (start 100 79.25) (end 97.5 79.25) (width 0.5) (layer B.Cu) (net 11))
 (segment (start 97.385 79.365) (end 96 79.365) (width 0.5) (layer B.Cu) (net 11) (status 20))
 (segment (start 97.5 79.25) (end 97.385 79.365) (width 0.5) (layer B.Cu) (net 11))
 (via (at 87.75 82) (size 0.8) (drill 0.4) (layers F.Cu B.Cu) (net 15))
 (segment (start 89.6 81.885) (end 87.865 81.885) (width 0.5) (layer F.Cu) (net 15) (status 10))
 (segment (start 87.865 81.885) (end 87.75 82) (width 0.5) (layer F.Cu) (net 15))
 (segment (start 87.845 81.905) (end 87.75 82) (width 0.5) (layer B.Cu) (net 15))
 (segment (start 89.5 81.905) (end 87.845 81.905) (width 0.5) (layer B.Cu) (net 15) (status 10))
 (via (at 87.75 80.5) (size 0.8) (drill 0.4) (layers F.Cu B.Cu) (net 16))
 (segment (start 89.6 80.615) (end 87.865 80.615) (width 0.5) (layer F.Cu) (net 16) (status 10))
 (segment (start 87.865 80.615) (end 87.75 80.5) (width 0.5) (layer F.Cu) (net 16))
 (segment (start 87.885 80.635) (end 87.75 80.5) (width 0.5) (layer B.Cu) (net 16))
 (segment (start 89.5 80.635) (end 87.885 80.635) (width 0.5) (layer B.Cu) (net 16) (status 10))
 (segment (start 98.1775 80.635) (end 98.3125 80.5) (width 0.5) (layer B.Cu) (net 2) (status 30))
 (segment (start 96 80.635) (end 98.1775 80.635) (width 0.5) (layer B.Cu) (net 2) (status 30))
 (segment (start 98.3125 80.5625) (end 100.25 82.5) (width 0.5) (layer B.Cu) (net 2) (status 30))
 (segment (start 98.3125 80.5) (end 98.3125 80.5625) (width 0.5) (layer B.Cu) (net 2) (status 30))
 (segment (start 100.25 84.5) (end 100.25 82.5) (width 0.5) (layer B.Cu) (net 2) (status 30))
 (segment (start 96 80.635) (end 94.365 80.635) (width 0.5) (layer B.Cu) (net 2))
 (segment (start 90.63 87.797919) (end 91.25 87.177919) (width 0.5) (layer B.Cu) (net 2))
 (segment (start 90.63 89) (end 90.63 87.797919) (width 0.5) (layer B.Cu) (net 2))
 (segment (start 91.25 87.177919) (end 91.25 85.25) (width 0.5) (layer B.Cu) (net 2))
 (segment (start 94.25 81.75) (end 94.25 80.75) (width 0.5) (layer B.Cu) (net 2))
 (segment (start 94.25 82.25) (end 94.25 81.75) (width 0.5) (layer B.Cu) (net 2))
 (segment (start 91.25 85.25) (end 94.25 82.25) (width 0.5) (layer B.Cu) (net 2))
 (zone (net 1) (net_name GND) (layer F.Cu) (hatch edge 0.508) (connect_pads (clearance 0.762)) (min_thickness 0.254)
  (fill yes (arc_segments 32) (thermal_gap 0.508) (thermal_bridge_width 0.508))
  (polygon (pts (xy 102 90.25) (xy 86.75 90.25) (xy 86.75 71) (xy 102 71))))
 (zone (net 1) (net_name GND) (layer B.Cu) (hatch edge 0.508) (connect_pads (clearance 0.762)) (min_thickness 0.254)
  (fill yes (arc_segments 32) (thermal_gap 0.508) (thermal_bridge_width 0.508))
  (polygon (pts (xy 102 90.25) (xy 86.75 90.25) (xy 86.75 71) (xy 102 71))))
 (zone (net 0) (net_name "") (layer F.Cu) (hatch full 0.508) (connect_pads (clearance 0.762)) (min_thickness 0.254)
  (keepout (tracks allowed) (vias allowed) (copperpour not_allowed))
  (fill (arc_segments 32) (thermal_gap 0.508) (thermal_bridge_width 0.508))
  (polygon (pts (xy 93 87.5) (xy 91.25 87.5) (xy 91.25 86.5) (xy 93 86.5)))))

